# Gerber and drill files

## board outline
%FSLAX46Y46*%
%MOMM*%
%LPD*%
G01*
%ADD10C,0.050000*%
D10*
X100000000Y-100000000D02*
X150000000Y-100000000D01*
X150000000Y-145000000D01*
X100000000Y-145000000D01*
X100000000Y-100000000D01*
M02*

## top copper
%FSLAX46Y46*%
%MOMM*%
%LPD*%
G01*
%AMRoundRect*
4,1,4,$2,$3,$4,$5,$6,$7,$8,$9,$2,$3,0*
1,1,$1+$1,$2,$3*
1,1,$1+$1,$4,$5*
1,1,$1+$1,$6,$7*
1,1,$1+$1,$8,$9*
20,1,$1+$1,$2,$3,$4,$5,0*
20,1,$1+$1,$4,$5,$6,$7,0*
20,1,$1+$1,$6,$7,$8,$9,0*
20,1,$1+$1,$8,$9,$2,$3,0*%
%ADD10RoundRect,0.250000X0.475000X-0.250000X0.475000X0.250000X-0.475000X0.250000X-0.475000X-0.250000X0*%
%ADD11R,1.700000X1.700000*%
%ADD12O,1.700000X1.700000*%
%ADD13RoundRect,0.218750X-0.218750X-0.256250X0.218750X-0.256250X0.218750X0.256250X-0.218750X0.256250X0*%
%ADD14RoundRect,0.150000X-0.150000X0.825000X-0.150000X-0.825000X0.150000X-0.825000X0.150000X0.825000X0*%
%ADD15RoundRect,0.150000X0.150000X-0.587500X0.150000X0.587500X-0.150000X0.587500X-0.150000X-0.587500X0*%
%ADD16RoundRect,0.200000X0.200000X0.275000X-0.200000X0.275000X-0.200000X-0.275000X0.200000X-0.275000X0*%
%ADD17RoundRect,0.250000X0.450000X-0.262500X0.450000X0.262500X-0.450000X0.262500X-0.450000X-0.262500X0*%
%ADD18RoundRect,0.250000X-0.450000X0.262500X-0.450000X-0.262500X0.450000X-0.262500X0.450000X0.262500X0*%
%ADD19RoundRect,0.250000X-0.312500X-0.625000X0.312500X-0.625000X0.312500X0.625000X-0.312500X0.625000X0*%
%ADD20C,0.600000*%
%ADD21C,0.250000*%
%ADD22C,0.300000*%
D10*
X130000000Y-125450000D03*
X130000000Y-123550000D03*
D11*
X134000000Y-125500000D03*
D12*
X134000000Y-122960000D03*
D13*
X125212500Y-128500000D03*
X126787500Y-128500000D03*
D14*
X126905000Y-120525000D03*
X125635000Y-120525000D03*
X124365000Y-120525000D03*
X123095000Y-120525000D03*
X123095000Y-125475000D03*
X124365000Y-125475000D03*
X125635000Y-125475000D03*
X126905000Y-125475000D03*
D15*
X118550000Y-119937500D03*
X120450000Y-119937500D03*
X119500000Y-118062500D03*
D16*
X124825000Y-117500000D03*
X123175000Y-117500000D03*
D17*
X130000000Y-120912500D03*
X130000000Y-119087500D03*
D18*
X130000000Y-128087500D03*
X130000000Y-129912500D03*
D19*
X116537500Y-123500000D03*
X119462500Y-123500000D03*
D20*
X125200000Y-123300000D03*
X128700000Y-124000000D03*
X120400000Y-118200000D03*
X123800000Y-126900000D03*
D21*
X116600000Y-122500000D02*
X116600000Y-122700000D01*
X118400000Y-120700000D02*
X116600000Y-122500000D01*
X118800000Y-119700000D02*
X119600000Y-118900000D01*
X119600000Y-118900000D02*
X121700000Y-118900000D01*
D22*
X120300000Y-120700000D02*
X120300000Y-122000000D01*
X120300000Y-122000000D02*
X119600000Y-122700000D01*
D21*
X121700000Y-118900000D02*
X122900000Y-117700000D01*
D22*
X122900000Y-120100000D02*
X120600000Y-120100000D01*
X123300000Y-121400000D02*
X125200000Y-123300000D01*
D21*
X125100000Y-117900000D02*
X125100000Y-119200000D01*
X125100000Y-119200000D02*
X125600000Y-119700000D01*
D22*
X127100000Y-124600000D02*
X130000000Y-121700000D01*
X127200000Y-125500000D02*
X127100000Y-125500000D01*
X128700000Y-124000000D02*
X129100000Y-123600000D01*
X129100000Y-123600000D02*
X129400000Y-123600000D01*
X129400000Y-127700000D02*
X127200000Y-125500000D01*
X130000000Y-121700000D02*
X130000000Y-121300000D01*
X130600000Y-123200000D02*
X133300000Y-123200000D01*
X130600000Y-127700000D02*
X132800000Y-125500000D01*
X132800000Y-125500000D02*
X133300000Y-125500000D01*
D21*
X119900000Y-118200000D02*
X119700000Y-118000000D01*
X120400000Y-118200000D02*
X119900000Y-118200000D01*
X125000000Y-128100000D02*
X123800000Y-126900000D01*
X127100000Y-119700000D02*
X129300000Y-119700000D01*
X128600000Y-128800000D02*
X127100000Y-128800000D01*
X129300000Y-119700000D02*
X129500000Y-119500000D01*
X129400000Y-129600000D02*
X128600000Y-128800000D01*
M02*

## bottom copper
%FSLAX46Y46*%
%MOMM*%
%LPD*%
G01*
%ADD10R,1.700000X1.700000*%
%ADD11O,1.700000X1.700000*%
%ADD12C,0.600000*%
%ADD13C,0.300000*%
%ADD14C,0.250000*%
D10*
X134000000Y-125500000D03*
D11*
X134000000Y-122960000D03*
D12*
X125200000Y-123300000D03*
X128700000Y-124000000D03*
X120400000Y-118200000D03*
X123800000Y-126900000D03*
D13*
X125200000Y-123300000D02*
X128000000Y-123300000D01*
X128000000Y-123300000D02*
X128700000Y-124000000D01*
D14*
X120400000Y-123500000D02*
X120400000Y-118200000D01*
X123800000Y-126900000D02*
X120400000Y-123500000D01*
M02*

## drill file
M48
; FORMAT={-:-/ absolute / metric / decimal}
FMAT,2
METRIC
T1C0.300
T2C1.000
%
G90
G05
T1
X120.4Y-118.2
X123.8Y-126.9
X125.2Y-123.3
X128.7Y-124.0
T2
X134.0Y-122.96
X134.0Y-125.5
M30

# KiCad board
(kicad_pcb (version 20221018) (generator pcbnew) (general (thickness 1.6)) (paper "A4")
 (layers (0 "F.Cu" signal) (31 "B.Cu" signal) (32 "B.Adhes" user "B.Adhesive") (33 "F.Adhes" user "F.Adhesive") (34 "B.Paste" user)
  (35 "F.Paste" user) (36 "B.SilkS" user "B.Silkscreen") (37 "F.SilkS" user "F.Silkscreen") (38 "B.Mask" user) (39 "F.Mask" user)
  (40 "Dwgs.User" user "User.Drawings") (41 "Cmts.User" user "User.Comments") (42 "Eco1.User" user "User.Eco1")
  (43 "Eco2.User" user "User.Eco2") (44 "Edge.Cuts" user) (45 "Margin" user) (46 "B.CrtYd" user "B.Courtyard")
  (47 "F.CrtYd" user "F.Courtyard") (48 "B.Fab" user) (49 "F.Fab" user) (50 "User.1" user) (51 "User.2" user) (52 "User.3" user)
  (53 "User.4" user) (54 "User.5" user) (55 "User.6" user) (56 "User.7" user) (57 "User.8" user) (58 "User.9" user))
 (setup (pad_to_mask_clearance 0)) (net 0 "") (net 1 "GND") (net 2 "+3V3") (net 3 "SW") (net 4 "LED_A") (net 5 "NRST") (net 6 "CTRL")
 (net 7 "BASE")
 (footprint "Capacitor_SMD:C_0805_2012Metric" (layer "F.Cu") (at 130 124.5 90)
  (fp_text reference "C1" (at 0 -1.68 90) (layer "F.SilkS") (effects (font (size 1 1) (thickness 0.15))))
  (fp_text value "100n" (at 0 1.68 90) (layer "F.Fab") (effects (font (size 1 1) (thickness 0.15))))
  (pad "1" smd roundrect (at -0.95 0 90) (size 1 1.45) (layers "F.Cu" "F.Paste" "F.Mask") (roundrect_rratio 0.25))
  (pad "2" smd roundrect (at 0.95 0 90) (size 1 1.45) (layers "F.Cu" "F.Paste" "F.Mask") (roundrect_rratio 0.25) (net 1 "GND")))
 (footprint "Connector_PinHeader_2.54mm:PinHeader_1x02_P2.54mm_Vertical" (layer "F.Cu") (at 134 125.5 180)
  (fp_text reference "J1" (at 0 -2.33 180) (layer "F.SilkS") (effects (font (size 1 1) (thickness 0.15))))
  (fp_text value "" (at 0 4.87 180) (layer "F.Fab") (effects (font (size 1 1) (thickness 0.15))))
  (pad "1" thru_hole rect (at 0 0 180) (size 1.7 1.7) (drill 1) (layers "*.Cu" "*.Mask") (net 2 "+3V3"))
  (pad "2" thru_hole oval (at 0 2.54 180) (size 1.7 1.7) (drill 1) (layers "*.Cu" "*.Mask") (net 1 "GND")))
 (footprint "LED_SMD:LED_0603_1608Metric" (layer "F.Cu") (at 126 128.5)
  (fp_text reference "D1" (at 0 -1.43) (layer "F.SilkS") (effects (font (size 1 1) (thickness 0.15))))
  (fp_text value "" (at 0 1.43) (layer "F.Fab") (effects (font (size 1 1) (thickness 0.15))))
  (pad "1" smd roundrect (at -0.7875 0) (size 0.875 0.95) (layers "F.Cu" "F.Paste" "F.Mask") (roundrect_rratio 0.25) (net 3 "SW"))
  (pad "2" smd roundrect (at 0.7875 0) (size 0.875 0.95) (layers "F.Cu" "F.Paste" "F.Mask") (roundrect_rratio 0.25) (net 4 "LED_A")))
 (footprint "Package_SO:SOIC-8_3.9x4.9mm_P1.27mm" (layer "F.Cu") (at 125 123 -90)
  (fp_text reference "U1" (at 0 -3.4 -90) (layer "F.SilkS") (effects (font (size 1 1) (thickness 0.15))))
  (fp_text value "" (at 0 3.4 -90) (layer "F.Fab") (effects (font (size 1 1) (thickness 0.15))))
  (pad "1" smd roundrect (at -2.475 -1.905 270) (size 1.95 0.6) (layers "F.Cu" "F.Paste" "F.Mask") (roundrect_rratio 0.25) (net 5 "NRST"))
  (pad "2" smd roundrect (at -2.475 -0.635 270) (size 1.95 0.6) (layers "F.Cu" "F.Paste" "F.Mask") (roundrect_rratio 0.25) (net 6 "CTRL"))
  (pad "3" smd roundrect (at -2.475 0.635 270) (size 1.95 0.6) (layers "F.Cu" "F.Paste" "F.Mask") (roundrect_rratio 0.25))
  (pad "4" smd roundrect (at -2.475 1.905 270) (size 1.95 0.6) (layers "F.Cu" "F.Paste" "F.Mask") (roundrect_rratio 0.25) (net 1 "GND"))
  (pad "5" smd roundrect (at 2.475 1.905 270) (size 1.95 0.6) (layers "F.Cu" "F.Paste" "F.Mask") (roundrect_rratio 0.25))
  (pad "6" smd roundrect (at 2.475 0.635 270) (size 1.95 0.6) (layers "F.Cu" "F.Paste" "F.Mask") (roundrect_rratio 0.25))
  (pad "7" smd roundrect (at 2.475 -0.635 270) (size 1.95 0.6) (layers "F.Cu" "F.Paste" "F.Mask") (roundrect_rratio 0.25))
  (pad "8" smd roundrect (at 2.475 -1.905 270) (size 1.95 0.6) (layers "F.Cu" "F.Paste" "F.Mask") (roundrect_rratio 0.25) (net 2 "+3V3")))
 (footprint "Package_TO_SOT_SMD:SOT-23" (layer "F.Cu") (at 119.5 119 90)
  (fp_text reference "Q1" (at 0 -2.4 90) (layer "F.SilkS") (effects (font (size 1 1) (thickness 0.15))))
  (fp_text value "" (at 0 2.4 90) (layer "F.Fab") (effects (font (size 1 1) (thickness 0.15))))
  (pad "1" smd roundrect (at -0.9375 -0.95 90) (size 1.475 0.6) (layers "F.Cu" "F.Paste" "F.Mask") (roundrect_rratio 0.25) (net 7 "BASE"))
  (pad "2" smd roundrect (at -0.9375 0.95 90) (size 1.475 0.6) (layers "F.Cu" "F.Paste" "F.Mask") (roundrect_rratio 0.25) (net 1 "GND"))
  (pad "3" smd roundrect (at 0.9375 0 90) (size 1.475 0.6) (layers "F.Cu" "F.Paste" "F.Mask") (roundrect_rratio 0.25) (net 3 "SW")))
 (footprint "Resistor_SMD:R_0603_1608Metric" (layer "F.Cu") (at 124 117.5 180)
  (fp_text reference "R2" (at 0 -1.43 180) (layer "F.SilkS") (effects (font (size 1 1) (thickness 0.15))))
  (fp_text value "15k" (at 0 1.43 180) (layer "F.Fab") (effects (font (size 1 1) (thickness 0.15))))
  (pad "1" smd roundrect (at -0.825 0 180) (size 0.8 0.95) (layers "F.Cu" "F.Paste" "F.Mask") (roundrect_rratio 0.25) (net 6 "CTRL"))
  (pad "2" smd roundrect (at 0.825 0 180) (size 0.8 0.95) (layers "F.Cu" "F.Paste" "F.Mask") (roundrect_rratio 0.25) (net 7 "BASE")))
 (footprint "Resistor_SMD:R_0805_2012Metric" (layer "F.Cu") (at 130 120 90)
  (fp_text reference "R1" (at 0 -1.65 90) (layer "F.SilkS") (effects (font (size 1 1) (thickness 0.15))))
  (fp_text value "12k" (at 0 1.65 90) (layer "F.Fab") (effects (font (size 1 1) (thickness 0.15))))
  (pad "1" smd roundrect (at -0.9125 0 90) (size 1.025 1.4) (layers "F.Cu" "F.Paste" "F.Mask") (roundrect_rratio 0.243902) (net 2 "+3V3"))
  (pad "2" smd roundrect (at 0.9125 0 90) (size 1.025 1.4) (layers "F.Cu" "F.Paste" "F.Mask") (roundrect_rratio 0.243902) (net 5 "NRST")))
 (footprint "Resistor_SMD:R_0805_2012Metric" (layer "F.Cu") (at 130 129 -90)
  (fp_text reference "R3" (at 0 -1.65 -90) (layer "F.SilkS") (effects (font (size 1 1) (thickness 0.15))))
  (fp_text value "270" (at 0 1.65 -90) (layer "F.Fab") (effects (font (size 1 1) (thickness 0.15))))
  (pad "1" smd roundrect (at -0.9125 0 270) (size 1.025 1.4) (layers "F.Cu" "F.Paste" "F.Mask") (roundrect_rratio 0.243902) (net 2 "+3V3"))
  (pad "2" smd roundrect (at 0.9125 0 270) (size 1.025 1.4) (layers "F.Cu" "F.Paste" "F.Mask") (roundrect_rratio 0.243902) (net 4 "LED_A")))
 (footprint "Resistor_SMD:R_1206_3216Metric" (layer "F.Cu") (at 118 123.5)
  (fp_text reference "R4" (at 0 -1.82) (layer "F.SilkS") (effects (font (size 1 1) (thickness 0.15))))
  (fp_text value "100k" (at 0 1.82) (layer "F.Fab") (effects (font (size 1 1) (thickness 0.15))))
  (pad "1" smd roundrect (at -1.4625 0) (size 1.125 1.75) (layers "F.Cu" "F.Paste" "F.Mask") (roundrect_rratio 0.222222) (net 7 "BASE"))
  (pad "2" smd roundrect (at 1.4625 0) (size 1.125 1.75) (layers "F.Cu" "F.Paste" "F.Mask") (roundrect_rratio 0.222222) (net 1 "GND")))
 (gr_rect (start 100 100) (end 150 145) (stroke (width 0.05) (type default)) (fill none) (layer "Edge.Cuts"))
 (segment (start 116.6 122.5) (end 116.6 122.7) (width 0.25) (layer "F.Cu") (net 7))
 (segment (start 118.4 120.7) (end 116.6 122.5) (width 0.25) (layer "F.Cu") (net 7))
 (segment (start 118.8 119.7) (end 119.6 118.9) (width 0.25) (layer "F.Cu") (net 7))
 (segment (start 119.6 118.9) (end 121.7 118.9) (width 0.25) (layer "F.Cu") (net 7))
 (segment (start 120.3 120.7) (end 120.3 122) (width 0.3) (layer "F.Cu") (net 1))
 (segment (start 120.3 122) (end 119.6 122.7) (width 0.3) (layer "F.Cu") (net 1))
 (segment (start 121.7 118.9) (end 122.9 117.7) (width 0.25) (layer "F.Cu") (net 7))
 (segment (start 122.9 120.1) (end 120.6 120.1) (width 0.3) (layer "F.Cu") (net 1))
 (segment (start 123.3 121.4) (end 125.2 123.3) (width 0.3) (layer "F.Cu") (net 1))
 (segment (start 125.1 117.9) (end 125.1 119.2) (width 0.25) (layer "F.Cu") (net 6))
 (segment (start 125.1 119.2) (end 125.6 119.7) (width 0.25) (layer "F.Cu") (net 6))
 (segment (start 127.1 124.6) (end 130 121.7) (width 0.3) (layer "F.Cu") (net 2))
 (segment (start 127.2 125.5) (end 127.1 125.5) (width 0.3) (layer "F.Cu") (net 2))
 (segment (start 128.7 124) (end 129.1 123.6) (width 0.3) (layer "F.Cu") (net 1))
 (segment (start 129.1 123.6) (end 129.4 123.6) (width 0.3) (layer "F.Cu") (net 1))
 (segment (start 129.4 127.7) (end 127.2 125.5) (width 0.3) (layer "F.Cu") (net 2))
 (segment (start 130 121.7) (end 130 121.3) (width 0.3) (layer "F.Cu") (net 2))
 (segment (start 130.6 123.2) (end 133.3 123.2) (width 0.3) (layer "F.Cu") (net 1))
 (segment (start 130.6 127.7) (end 132.8 125.5) (width 0.3) (layer "F.Cu") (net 2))
 (segment (start 132.8 125.5) (end 133.3 125.5) (width 0.3) (layer "F.Cu") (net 2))
 (via (at 125.2 123.3) (size 0.6) (drill 0.3) (layers "F.Cu" "B.Cu") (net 1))
 (via (at 128.7 124) (size 0.6) (drill 0.3) (layers "F.Cu" "B.Cu") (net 1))
 (segment (start 119.9 118.2) (end 119.7 118) (width 0.25) (layer "F.Cu") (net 3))
 (segment (start 120.4 118.2) (end 119.9 118.2) (width 0.25) (layer "F.Cu") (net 3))
 (segment (start 125 128.1) (end 123.8 126.9) (width 0.25) (layer "F.Cu") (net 3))
 (segment (start 125.2 123.3) (end 128 123.3) (width 0.3) (layer "B.Cu") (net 1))
 (segment (start 127.1 119.7) (end 129.3 119.7) (width 0.25) (layer "F.Cu") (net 5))
 (segment (start 128 123.3) (end 128.7 124) (width 0.3) (layer "B.Cu") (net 1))
 (segment (start 128.6 128.8) (end 127.1 128.8) (width 0.25) (layer "F.Cu") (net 4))
 (segment (start 129.3 119.7) (end 129.5 119.5) (width 0.25) (layer "F.Cu") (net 5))
 (segment (start 129.4 129.6) (end 128.6 128.8) (width 0.25) (layer "F.Cu") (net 4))
 (via (at 120.4 118.2) (size 0.6) (drill 0.3) (layers "F.Cu" "B.Cu") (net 3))
 (via (at 123.8 126.9) (size 0.6) (drill 0.3) (layers "F.Cu" "B.Cu") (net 3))
 (segment (start 120.4 123.5) (end 120.4 118.2) (width 0.25) (layer "B.Cu") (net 3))
 (segment (start 123.8 126.9) (end 120.4 123.5) (width 0.25) (layer "B.Cu") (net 3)))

